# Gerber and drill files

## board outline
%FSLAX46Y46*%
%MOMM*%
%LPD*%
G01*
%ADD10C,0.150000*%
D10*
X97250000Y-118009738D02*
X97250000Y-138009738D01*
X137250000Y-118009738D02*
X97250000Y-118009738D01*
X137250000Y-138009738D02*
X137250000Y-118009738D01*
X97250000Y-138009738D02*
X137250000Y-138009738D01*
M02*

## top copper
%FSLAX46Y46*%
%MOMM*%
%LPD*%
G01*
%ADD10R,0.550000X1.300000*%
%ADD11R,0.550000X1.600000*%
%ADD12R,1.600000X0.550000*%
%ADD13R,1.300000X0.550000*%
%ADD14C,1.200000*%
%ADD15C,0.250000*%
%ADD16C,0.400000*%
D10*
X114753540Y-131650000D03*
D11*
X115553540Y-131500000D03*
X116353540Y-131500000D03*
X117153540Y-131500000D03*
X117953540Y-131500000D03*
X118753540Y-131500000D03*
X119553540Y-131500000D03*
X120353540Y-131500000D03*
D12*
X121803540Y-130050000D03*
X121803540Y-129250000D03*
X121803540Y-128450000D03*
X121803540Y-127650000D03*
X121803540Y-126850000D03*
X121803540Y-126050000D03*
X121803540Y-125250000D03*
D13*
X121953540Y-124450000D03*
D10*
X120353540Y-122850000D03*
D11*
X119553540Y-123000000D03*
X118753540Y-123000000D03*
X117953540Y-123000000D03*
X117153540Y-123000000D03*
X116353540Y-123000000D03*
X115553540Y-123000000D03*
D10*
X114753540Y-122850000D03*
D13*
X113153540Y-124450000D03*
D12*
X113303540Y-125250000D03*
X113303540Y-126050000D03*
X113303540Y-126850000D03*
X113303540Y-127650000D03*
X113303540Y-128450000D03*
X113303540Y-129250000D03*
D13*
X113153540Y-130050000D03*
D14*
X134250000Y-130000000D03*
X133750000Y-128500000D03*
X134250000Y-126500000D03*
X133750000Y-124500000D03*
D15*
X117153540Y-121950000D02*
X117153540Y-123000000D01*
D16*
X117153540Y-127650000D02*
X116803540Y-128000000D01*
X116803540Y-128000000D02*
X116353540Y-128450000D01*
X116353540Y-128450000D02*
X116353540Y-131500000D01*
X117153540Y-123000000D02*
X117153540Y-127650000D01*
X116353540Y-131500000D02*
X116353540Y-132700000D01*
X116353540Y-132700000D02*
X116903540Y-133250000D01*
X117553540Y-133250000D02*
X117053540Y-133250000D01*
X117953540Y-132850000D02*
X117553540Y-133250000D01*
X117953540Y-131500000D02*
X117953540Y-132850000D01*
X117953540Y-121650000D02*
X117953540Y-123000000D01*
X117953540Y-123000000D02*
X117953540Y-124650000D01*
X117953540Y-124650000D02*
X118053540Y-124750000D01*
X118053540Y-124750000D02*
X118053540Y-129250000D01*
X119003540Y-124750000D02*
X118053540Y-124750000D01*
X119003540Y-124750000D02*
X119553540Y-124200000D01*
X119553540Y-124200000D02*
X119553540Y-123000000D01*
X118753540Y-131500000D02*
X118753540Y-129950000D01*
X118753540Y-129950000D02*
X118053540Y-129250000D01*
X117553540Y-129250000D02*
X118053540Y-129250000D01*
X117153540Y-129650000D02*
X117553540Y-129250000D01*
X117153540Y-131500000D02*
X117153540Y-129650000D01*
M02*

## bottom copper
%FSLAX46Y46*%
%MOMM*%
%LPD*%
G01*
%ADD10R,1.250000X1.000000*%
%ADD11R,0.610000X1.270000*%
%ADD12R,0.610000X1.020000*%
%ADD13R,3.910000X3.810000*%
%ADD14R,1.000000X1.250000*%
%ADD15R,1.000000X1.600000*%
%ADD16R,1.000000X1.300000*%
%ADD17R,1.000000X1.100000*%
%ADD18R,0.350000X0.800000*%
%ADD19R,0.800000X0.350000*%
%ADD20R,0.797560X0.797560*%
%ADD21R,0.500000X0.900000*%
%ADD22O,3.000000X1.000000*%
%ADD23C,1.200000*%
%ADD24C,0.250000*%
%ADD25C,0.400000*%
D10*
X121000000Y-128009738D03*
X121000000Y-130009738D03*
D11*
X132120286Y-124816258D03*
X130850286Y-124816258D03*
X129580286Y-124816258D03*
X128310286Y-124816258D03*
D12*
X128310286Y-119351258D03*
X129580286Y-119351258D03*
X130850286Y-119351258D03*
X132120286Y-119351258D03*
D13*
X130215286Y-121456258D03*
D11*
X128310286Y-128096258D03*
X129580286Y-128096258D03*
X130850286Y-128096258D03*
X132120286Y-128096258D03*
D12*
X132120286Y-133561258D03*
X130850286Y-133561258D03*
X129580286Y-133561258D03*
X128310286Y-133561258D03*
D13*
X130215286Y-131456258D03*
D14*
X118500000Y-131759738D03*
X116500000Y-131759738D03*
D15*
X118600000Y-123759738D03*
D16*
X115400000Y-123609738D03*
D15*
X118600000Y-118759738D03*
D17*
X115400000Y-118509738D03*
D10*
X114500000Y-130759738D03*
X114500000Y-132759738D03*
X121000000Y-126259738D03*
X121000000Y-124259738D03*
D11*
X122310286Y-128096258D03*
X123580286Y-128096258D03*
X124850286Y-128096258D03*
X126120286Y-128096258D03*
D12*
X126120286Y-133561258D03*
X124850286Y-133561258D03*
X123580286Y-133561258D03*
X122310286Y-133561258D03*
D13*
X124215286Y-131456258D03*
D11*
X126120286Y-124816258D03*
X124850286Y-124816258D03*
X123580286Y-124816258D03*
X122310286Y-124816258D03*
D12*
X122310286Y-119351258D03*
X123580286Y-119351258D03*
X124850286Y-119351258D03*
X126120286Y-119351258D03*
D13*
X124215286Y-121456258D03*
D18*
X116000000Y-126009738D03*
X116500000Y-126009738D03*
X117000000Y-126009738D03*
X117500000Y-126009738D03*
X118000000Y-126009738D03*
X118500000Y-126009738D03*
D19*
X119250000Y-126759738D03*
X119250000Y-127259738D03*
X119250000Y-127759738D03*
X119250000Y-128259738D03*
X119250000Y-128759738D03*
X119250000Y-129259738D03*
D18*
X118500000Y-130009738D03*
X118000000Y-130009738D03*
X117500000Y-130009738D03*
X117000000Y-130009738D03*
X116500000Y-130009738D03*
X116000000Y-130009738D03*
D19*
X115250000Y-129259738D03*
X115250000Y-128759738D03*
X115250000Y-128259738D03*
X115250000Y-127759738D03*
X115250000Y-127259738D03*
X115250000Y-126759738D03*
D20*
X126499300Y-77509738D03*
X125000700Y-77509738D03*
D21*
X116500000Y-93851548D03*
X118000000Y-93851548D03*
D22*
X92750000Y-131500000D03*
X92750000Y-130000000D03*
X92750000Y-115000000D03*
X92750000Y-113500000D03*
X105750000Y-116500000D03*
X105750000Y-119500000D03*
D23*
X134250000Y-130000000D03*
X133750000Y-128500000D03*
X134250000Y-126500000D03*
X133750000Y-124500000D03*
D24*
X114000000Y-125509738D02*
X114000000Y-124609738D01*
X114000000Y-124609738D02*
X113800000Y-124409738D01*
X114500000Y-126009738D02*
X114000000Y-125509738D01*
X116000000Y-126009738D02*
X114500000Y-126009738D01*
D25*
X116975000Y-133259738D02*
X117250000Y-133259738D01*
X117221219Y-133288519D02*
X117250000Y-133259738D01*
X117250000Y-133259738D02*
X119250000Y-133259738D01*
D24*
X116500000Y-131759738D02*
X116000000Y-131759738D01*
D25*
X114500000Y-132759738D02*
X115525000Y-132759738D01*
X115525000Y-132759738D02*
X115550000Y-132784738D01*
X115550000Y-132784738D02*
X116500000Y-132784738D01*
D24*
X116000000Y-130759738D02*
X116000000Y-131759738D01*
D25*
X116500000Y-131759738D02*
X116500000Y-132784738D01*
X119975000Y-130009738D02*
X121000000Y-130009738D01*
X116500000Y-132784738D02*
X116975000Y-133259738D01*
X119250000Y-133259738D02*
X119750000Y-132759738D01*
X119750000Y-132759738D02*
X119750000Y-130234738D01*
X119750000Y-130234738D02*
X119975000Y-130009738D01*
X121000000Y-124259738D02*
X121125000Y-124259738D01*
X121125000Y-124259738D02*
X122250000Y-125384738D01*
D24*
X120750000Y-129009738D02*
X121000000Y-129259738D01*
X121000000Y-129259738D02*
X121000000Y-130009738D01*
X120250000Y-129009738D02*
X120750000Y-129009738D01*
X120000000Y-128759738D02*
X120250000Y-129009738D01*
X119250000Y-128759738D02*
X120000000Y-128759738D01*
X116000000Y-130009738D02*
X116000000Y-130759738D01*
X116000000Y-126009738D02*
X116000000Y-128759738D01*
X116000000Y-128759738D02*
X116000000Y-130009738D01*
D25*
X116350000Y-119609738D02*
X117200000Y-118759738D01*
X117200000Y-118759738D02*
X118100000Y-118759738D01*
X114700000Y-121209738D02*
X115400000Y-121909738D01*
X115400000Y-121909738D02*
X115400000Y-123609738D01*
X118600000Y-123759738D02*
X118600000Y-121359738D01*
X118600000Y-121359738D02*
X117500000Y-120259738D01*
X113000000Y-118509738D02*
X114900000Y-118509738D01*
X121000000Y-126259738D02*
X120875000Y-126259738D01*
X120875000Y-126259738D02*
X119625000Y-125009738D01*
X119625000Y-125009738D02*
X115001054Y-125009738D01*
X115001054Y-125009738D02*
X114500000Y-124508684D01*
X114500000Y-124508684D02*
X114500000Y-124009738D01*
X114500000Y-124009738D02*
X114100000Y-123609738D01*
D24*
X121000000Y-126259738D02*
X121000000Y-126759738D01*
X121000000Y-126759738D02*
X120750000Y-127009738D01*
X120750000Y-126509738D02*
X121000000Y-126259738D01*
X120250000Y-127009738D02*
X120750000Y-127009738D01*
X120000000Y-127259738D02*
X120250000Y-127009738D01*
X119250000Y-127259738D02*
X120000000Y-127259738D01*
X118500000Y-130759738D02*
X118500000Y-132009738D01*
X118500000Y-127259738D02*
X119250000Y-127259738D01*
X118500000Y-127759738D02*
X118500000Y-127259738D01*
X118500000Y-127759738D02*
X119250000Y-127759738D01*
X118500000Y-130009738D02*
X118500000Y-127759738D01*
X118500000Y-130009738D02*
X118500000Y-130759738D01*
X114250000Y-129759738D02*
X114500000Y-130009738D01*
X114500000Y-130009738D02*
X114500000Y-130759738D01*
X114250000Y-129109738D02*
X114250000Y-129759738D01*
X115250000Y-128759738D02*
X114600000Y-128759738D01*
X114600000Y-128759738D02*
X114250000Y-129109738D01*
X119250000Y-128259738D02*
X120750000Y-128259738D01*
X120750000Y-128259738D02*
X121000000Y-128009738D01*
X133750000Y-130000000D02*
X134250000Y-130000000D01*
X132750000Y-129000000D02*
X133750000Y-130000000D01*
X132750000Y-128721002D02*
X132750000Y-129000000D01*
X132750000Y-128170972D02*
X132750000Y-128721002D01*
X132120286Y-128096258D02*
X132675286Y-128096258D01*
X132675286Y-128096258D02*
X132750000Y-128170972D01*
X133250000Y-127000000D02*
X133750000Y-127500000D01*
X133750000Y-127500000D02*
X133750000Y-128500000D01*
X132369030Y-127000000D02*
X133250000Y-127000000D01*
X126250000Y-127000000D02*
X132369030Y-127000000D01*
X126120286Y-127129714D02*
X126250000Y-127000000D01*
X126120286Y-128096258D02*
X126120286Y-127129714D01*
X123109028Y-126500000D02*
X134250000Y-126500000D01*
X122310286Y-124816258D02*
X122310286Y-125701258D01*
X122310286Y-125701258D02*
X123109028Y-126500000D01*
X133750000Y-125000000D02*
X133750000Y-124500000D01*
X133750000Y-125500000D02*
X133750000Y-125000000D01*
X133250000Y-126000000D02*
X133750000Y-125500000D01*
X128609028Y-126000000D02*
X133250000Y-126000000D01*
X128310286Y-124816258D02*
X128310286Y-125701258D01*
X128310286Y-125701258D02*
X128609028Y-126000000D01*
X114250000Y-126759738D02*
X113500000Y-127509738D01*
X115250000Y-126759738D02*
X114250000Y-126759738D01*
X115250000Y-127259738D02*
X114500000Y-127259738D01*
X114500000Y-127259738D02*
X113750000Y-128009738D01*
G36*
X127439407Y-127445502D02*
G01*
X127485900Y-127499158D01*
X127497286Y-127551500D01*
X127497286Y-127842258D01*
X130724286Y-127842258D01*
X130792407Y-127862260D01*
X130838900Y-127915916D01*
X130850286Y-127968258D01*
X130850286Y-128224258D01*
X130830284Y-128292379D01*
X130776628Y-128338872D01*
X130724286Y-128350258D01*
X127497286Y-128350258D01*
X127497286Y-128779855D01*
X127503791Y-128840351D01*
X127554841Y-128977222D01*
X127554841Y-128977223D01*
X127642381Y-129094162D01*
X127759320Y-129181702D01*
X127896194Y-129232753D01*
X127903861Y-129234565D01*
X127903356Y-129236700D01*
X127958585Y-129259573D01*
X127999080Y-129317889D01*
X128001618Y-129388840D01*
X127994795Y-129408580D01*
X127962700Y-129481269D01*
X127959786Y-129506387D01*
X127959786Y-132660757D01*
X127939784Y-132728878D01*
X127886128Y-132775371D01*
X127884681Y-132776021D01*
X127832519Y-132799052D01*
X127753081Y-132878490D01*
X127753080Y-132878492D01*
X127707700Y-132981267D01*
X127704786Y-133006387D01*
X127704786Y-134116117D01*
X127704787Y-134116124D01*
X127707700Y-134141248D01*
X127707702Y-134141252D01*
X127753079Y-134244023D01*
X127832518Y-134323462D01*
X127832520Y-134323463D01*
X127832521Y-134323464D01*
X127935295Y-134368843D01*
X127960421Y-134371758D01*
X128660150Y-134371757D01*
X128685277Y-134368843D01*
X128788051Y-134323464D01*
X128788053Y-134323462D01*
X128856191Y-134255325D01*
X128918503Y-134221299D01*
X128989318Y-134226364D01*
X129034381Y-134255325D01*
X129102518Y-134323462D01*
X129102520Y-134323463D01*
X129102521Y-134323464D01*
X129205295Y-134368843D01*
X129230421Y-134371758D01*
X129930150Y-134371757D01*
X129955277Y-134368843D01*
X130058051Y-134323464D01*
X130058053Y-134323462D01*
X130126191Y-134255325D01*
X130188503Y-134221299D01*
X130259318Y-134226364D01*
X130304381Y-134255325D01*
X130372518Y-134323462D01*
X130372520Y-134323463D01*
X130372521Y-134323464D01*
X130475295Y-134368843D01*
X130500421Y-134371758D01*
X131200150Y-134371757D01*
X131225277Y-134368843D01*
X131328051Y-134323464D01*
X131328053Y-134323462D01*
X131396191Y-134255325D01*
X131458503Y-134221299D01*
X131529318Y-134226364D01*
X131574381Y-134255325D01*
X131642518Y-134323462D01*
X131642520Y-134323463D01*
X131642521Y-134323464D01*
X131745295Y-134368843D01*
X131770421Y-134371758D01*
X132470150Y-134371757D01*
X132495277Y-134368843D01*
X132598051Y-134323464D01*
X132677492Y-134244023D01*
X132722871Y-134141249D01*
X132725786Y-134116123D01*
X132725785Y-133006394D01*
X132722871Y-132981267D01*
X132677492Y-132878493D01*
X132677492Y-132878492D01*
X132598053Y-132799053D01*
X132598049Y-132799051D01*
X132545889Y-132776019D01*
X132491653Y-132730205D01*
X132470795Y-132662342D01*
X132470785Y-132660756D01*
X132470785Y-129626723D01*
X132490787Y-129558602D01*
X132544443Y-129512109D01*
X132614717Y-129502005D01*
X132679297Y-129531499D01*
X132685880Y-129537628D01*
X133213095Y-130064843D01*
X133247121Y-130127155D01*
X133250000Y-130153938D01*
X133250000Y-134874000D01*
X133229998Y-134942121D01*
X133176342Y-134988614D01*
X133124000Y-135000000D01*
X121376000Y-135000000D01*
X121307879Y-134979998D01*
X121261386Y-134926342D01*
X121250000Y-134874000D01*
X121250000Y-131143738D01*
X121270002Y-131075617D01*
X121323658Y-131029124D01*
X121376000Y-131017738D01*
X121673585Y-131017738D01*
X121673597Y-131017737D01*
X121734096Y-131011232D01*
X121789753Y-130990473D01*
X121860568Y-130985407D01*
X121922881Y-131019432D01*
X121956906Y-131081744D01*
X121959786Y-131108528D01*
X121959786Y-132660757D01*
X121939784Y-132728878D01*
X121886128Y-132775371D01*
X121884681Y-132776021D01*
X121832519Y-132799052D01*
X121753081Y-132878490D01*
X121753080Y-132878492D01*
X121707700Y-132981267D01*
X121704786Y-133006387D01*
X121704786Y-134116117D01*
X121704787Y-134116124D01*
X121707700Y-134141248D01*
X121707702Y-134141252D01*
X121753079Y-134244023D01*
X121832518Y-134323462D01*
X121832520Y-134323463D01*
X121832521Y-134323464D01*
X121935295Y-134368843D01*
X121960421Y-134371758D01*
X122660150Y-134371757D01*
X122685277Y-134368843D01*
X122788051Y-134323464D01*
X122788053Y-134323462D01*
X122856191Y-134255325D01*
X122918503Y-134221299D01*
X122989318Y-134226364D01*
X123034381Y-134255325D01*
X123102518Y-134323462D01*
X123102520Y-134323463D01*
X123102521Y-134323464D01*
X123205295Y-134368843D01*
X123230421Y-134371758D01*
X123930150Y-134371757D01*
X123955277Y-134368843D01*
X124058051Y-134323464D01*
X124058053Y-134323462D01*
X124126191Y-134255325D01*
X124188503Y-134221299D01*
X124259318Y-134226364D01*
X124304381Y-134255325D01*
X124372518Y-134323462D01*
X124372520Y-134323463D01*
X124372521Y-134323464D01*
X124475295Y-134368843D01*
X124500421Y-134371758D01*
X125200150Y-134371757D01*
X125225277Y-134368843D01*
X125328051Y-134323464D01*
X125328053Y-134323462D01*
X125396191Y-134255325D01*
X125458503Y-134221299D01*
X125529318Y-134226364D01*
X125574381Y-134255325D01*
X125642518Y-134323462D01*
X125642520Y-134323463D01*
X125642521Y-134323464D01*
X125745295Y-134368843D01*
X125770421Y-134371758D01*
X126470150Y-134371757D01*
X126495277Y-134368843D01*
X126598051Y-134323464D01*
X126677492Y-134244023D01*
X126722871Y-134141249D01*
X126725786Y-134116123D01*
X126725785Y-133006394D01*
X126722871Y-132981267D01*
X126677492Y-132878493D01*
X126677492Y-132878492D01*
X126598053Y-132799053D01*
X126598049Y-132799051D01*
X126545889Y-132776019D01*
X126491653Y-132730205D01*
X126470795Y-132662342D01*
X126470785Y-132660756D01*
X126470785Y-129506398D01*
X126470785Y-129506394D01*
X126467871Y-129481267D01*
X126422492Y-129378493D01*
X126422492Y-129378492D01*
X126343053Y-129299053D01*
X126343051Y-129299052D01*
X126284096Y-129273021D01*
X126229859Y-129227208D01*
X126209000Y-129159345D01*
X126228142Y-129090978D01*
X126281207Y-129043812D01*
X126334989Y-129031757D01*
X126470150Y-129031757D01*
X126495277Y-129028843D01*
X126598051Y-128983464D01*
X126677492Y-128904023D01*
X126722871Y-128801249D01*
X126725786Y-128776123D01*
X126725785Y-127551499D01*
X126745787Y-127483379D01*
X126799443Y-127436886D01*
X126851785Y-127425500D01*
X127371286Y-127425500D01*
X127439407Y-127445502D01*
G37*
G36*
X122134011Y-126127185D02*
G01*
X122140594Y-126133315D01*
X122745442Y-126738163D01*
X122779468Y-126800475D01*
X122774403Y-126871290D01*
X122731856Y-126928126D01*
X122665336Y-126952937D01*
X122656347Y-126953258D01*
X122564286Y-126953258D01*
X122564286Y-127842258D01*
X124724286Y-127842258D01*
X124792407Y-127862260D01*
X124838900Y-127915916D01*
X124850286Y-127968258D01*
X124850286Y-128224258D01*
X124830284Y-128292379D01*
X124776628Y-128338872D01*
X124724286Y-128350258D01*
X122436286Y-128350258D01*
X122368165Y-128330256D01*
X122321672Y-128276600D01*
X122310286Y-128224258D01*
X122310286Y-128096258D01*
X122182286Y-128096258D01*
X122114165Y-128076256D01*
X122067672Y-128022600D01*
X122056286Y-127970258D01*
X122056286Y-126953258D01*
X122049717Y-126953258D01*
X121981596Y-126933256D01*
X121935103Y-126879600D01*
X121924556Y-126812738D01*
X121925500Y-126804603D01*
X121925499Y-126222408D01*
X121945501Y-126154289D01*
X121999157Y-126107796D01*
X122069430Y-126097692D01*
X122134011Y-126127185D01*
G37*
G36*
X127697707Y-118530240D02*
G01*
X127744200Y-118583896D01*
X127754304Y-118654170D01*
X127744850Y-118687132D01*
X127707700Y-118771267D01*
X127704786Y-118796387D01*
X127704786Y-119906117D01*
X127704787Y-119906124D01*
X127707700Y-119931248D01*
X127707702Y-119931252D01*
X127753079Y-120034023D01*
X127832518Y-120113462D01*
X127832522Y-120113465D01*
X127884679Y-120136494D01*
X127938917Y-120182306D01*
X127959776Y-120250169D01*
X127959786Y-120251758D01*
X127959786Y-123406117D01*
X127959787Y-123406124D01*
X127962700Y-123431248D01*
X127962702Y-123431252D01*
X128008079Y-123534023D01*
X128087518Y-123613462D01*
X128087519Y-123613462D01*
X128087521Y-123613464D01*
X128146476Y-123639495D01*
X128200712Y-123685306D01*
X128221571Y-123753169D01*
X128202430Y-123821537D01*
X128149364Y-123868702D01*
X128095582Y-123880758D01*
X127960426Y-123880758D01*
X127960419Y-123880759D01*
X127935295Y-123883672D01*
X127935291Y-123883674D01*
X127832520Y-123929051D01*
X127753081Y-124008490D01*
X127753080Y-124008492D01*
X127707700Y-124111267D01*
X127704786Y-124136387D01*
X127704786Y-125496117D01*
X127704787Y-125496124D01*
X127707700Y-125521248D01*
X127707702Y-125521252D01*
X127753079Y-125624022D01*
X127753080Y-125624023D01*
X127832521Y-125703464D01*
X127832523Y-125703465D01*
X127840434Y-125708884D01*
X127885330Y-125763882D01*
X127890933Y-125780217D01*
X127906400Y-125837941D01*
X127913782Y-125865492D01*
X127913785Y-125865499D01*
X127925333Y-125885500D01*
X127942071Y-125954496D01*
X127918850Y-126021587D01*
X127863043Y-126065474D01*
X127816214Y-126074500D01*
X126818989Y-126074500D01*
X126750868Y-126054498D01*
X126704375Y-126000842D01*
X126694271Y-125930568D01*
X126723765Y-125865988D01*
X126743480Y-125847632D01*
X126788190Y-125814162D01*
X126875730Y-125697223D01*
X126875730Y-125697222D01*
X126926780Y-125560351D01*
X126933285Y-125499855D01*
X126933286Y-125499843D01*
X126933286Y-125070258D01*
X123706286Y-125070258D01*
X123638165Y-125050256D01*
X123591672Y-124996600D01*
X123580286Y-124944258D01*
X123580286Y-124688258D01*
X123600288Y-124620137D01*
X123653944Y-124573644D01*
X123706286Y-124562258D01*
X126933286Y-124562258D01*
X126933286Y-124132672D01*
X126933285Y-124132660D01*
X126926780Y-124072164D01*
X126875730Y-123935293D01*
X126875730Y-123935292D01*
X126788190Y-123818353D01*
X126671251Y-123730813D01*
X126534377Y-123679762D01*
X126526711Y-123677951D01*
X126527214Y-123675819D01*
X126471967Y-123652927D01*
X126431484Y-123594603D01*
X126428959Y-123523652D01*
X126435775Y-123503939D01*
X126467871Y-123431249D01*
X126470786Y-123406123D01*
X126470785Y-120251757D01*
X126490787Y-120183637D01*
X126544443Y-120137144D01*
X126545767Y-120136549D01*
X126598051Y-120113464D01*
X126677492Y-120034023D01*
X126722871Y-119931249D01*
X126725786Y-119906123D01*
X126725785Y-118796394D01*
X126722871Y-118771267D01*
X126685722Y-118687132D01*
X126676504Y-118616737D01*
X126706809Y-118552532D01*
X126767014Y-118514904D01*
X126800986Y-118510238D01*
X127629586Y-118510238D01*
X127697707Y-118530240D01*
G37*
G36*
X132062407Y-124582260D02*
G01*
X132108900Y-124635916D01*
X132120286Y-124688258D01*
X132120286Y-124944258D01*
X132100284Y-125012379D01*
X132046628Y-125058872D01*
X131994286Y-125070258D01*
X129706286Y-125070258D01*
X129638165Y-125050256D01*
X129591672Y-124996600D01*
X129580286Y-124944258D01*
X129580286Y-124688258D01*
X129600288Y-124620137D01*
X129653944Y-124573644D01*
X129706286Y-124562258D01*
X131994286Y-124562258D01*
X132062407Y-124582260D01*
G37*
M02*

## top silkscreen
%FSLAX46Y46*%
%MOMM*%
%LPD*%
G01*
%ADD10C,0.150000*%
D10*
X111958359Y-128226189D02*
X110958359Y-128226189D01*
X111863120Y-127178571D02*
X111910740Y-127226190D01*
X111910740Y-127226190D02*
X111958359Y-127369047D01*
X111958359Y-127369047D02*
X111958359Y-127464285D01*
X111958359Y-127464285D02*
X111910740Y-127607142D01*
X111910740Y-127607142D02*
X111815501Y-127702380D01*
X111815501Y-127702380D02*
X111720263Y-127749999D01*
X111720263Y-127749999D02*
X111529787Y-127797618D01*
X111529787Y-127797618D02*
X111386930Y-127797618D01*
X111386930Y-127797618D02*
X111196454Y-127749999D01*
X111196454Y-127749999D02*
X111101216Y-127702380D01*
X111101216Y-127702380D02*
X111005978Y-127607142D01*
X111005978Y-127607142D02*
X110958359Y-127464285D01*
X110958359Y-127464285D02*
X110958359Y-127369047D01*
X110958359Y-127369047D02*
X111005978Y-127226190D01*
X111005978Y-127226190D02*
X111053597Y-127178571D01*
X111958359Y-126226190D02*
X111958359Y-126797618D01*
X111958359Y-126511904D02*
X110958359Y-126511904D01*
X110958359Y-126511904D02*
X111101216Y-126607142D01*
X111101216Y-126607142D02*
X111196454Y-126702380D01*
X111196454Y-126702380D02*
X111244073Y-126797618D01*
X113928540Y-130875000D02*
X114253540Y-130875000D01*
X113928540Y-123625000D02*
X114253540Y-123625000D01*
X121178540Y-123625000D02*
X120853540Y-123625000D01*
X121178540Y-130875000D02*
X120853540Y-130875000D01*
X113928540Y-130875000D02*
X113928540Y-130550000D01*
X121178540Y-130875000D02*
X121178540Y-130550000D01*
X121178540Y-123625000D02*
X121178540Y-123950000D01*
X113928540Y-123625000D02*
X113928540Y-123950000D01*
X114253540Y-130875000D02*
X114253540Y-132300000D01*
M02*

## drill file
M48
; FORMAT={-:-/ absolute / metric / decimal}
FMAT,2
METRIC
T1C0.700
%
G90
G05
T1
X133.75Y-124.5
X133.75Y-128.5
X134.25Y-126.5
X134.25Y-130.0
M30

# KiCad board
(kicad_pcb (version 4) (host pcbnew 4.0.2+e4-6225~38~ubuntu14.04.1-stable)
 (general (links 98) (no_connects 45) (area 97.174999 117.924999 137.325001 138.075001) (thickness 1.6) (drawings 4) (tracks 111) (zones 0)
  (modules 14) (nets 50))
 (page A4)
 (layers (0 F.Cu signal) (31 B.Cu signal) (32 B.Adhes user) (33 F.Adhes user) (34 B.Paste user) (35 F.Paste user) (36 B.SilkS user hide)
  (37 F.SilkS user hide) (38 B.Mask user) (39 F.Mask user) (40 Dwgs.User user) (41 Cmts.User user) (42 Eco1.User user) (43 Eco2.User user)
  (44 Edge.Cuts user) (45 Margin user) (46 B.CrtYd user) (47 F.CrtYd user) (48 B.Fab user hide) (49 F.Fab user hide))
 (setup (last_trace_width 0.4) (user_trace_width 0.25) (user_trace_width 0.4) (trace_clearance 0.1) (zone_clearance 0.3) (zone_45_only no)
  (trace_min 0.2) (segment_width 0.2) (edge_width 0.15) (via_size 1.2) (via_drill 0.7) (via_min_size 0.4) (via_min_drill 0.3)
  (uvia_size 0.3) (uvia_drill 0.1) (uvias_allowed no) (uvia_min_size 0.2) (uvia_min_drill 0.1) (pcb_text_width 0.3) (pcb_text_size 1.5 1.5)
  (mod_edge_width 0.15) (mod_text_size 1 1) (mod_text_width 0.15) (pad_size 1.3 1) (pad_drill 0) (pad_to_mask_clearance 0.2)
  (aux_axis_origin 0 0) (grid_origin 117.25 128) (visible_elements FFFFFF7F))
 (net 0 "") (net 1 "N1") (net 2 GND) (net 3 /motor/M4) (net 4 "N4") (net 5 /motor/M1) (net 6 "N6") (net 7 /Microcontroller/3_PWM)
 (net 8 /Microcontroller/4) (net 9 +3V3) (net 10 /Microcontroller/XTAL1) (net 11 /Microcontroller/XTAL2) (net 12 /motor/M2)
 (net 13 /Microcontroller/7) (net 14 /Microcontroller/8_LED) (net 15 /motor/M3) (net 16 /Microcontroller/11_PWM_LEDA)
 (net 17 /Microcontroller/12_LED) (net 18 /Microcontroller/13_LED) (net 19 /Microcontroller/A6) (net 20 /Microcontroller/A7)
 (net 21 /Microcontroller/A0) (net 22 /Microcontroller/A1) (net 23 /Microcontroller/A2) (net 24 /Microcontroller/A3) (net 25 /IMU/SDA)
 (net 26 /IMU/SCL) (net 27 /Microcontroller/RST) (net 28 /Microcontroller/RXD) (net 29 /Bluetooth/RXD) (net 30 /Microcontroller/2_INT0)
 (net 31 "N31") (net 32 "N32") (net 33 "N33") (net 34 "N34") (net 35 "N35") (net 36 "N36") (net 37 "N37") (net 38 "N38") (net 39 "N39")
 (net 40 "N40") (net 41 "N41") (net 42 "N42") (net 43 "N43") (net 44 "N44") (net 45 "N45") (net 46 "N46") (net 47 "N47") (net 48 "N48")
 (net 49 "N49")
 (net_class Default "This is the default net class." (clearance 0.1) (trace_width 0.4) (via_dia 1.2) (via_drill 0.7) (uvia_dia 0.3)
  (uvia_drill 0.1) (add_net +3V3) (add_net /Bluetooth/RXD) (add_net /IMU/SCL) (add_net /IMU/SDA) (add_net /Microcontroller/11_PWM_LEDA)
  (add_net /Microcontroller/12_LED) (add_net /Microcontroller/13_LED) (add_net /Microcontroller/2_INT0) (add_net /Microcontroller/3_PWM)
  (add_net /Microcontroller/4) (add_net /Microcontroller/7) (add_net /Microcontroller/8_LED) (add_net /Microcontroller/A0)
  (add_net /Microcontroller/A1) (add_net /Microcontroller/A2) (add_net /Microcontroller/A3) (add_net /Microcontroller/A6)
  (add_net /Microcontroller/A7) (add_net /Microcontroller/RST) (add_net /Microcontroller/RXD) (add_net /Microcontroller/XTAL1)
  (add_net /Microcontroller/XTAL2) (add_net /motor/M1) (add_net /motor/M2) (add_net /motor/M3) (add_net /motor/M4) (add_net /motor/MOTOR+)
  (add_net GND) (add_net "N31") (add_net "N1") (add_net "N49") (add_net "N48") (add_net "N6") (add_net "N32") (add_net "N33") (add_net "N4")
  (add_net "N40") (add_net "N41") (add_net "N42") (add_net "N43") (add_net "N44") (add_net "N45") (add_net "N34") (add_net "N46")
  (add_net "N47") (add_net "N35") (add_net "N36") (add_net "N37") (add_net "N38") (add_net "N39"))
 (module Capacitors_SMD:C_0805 (layer B.Cu) (at 121 129.009738 270)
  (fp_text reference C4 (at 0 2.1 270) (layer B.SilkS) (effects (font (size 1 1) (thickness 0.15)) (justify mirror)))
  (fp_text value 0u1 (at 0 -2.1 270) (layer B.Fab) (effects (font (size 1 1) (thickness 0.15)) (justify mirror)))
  (pad 1 smd rect (at -1 0 270) (size 1 1.25) (layers B.Cu B.Paste B.Mask) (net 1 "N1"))
  (pad 2 smd rect (at 1 0 270) (size 1 1.25) (layers B.Cu B.Paste B.Mask) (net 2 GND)))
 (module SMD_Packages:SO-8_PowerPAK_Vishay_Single (layer B.Cu) (at 130.215286 122.146258 90)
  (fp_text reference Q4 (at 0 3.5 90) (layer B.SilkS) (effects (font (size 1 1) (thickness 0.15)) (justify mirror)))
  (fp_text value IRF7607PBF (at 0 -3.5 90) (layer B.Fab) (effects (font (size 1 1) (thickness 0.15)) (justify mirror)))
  (pad 1 smd rect (at -2.67 1.905 90) (size 1.27 0.61) (layers B.Cu B.Paste B.Mask) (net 2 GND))
  (pad 2 smd rect (at -2.67 0.635 90) (size 1.27 0.61) (layers B.Cu B.Paste B.Mask) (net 2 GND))
  (pad 3 smd rect (at -2.67 -0.635 90) (size 1.27 0.61) (layers B.Cu B.Paste B.Mask) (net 2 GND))
  (pad 4 smd rect (at -2.67 -1.905 90) (size 1.27 0.61) (layers B.Cu B.Paste B.Mask) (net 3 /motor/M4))
  (pad 5 smd rect (at 2.795 -1.905 90) (size 1.02 0.61) (layers B.Cu B.Paste B.Mask) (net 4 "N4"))
  (pad 5 smd rect (at 2.795 -0.635 90) (size 1.02 0.61) (layers B.Cu B.Paste B.Mask) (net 4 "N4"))
  (pad 5 smd rect (at 2.795 0.635 90) (size 1.02 0.61) (layers B.Cu B.Paste B.Mask) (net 4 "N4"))
  (pad 5 smd rect (at 2.795 1.905 90) (size 1.02 0.61) (layers B.Cu B.Paste B.Mask) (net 4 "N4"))
  (pad 5 smd rect (at 0.69 0 90) (size 3.81 3.91) (layers B.Cu B.Paste B.Mask) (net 4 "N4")))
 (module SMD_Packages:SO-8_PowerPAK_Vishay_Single (layer B.Cu) (at 130.215286 130.766258 270)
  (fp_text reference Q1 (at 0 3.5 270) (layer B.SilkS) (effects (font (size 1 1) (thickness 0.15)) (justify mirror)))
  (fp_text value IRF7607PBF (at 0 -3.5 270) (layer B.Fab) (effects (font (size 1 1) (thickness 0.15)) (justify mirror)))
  (pad 1 smd rect (at -2.67 1.905 270) (size 1.27 0.61) (layers B.Cu B.Paste B.Mask) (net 2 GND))
  (pad 2 smd rect (at -2.67 0.635 270) (size 1.27 0.61) (layers B.Cu B.Paste B.Mask) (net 2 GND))
  (pad 3 smd rect (at -2.67 -0.635 270) (size 1.27 0.61) (layers B.Cu B.Paste B.Mask) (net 2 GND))
  (pad 4 smd rect (at -2.67 -1.905 270) (size 1.27 0.61) (layers B.Cu B.Paste B.Mask) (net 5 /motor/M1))
  (pad 5 smd rect (at 2.795 -1.905 270) (size 1.02 0.61) (layers B.Cu B.Paste B.Mask) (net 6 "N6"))
  (pad 5 smd rect (at 2.795 -0.635 270) (size 1.02 0.61) (layers B.Cu B.Paste B.Mask) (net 6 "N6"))
  (pad 5 smd rect (at 2.795 0.635 270) (size 1.02 0.61) (layers B.Cu B.Paste B.Mask) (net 6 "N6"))
  (pad 5 smd rect (at 2.795 1.905 270) (size 1.02 0.61) (layers B.Cu B.Paste B.Mask) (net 6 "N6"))
  (pad 5 smd rect (at 0.69 0 270) (size 3.81 3.91) (layers B.Cu B.Paste B.Mask) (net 6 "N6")))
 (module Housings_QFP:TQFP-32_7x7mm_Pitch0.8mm (layer F.Cu) (at 117.55354 127.25 90)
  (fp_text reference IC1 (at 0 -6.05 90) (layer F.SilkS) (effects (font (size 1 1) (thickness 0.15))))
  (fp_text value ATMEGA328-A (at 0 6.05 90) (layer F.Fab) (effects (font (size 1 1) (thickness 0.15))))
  (fp_line (start -3.625 -3.625) (end -3.625 -3.3) (layer F.SilkS) (width 0.15))
  (fp_line (start 3.625 -3.625) (end 3.625 -3.3) (layer F.SilkS) (width 0.15))
  (fp_line (start 3.625 3.625) (end 3.625 3.3) (layer F.SilkS) (width 0.15))
  (fp_line (start -3.625 3.625) (end -3.625 3.3) (layer F.SilkS) (width 0.15))
  (fp_line (start -3.625 -3.625) (end -3.3 -3.625) (layer F.SilkS) (width 0.15))
  (fp_line (start -3.625 3.625) (end -3.3 3.625) (layer F.SilkS) (width 0.15))
  (fp_line (start 3.625 3.625) (end 3.3 3.625) (layer F.SilkS) (width 0.15))
  (fp_line (start 3.625 -3.625) (end 3.3 -3.625) (layer F.SilkS) (width 0.15))
  (fp_line (start -3.625 -3.3) (end -5.05 -3.3) (layer F.SilkS) (width 0.15))
  (pad 1 smd rect (at -4.4 -2.8 90) (size 1.3 0.55) (layers F.Cu F.Paste F.Mask) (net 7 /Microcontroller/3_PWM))
  (pad 2 smd rect (at -4.25 -2 90) (size 1.6 0.55) (layers F.Cu F.Paste F.Mask) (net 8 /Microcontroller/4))
  (pad 3 smd rect (at -4.25 -1.2 90) (size 1.6 0.55) (layers F.Cu F.Paste F.Mask) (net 2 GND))
  (pad 4 smd rect (at -4.25 -0.4 90) (size 1.6 0.55) (layers F.Cu F.Paste F.Mask) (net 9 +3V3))
  (pad 5 smd rect (at -4.25 0.4 90) (size 1.6 0.55) (layers F.Cu F.Paste F.Mask) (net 2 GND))
  (pad 6 smd rect (at -4.25 1.2 90) (size 1.6 0.55) (layers F.Cu F.Paste F.Mask) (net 9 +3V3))
  (pad 7 smd rect (at -4.25 2 90) (size 1.6 0.55) (layers F.Cu F.Paste F.Mask) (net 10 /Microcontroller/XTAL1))
  (pad 8 smd rect (at -4.25 2.8 90) (size 1.6 0.55) (layers F.Cu F.Paste F.Mask) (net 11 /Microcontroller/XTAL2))
  (pad 9 smd rect (at -2.8 4.25 180) (size 1.6 0.55) (layers F.Cu F.Paste F.Mask) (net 5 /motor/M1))
  (pad 10 smd rect (at -2 4.25 180) (size 1.6 0.55) (layers F.Cu F.Paste F.Mask) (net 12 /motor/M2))
  (pad 11 smd rect (at -1.2 4.25 180) (size 1.6 0.55) (layers F.Cu F.Paste F.Mask) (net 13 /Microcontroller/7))
  (pad 12 smd rect (at -0.4 4.25 180) (size 1.6 0.55) (layers F.Cu F.Paste F.Mask) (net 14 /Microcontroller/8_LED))
  (pad 13 smd rect (at 0.4 4.25 180) (size 1.6 0.55) (layers F.Cu F.Paste F.Mask) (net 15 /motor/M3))
  (pad 14 smd rect (at 1.2 4.25 180) (size 1.6 0.55) (layers F.Cu F.Paste F.Mask) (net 3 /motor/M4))
  (pad 15 smd rect (at 2 4.25 180) (size 1.6 0.55) (layers F.Cu F.Paste F.Mask) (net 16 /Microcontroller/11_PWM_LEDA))
  (pad 16 smd rect (at 2.8 4.4 180) (size 1.3 0.55) (layers F.Cu F.Paste F.Mask) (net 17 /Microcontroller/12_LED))
  (pad 17 smd rect (at 4.4 2.8 90) (size 1.3 0.55) (layers F.Cu F.Paste F.Mask) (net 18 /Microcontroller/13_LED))
  (pad 18 smd rect (at 4.25 2 90) (size 1.6 0.55) (layers F.Cu F.Paste F.Mask) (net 9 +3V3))
  (pad 19 smd rect (at 4.25 1.2 90) (size 1.6 0.55) (layers F.Cu F.Paste F.Mask) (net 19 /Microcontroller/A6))
  (pad 20 smd rect (at 4.25 0.4 90) (size 1.6 0.55) (layers F.Cu F.Paste F.Mask) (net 9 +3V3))
  (pad 21 smd rect (at 4.25 -0.4 90) (size 1.6 0.55) (layers F.Cu F.Paste F.Mask) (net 2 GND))
  (pad 22 smd rect (at 4.25 -1.2 90) (size 1.6 0.55) (layers F.Cu F.Paste F.Mask) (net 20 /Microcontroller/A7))
  (pad 23 smd rect (at 4.25 -2 90) (size 1.6 0.55) (layers F.Cu F.Paste F.Mask) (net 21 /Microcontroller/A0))
  (pad 24 smd rect (at 4.4 -2.8 90) (size 1.3 0.55) (layers F.Cu F.Paste F.Mask) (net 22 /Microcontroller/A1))
  (pad 25 smd rect (at 2.8 -4.4 180) (size 1.3 0.55) (layers F.Cu F.Paste F.Mask) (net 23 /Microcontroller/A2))
  (pad 26 smd rect (at 2 -4.25 180) (size 1.6 0.55) (layers F.Cu F.Paste F.Mask) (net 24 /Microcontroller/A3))
  (pad 27 smd rect (at 1.2 -4.25 180) (size 1.6 0.55) (layers F.Cu F.Paste F.Mask) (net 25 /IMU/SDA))
  (pad 28 smd rect (at 0.4 -4.25 180) (size 1.6 0.55) (layers F.Cu F.Paste F.Mask) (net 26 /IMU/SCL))
  (pad 29 smd rect (at -0.4 -4.25 180) (size 1.6 0.55) (layers F.Cu F.Paste F.Mask) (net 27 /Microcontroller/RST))
  (pad 30 smd rect (at -1.2 -4.25 180) (size 1.6 0.55) (layers F.Cu F.Paste F.Mask) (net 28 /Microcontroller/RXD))
  (pad 31 smd rect (at -2 -4.25 180) (size 1.6 0.55) (layers F.Cu F.Paste F.Mask) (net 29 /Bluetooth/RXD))
  (pad 32 smd rect (at -2.8 -4.4 180) (size 1.3 0.55) (layers F.Cu F.Paste F.Mask) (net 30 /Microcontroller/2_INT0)))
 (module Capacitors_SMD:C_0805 (layer B.Cu) (at 117.5 131.759738 180)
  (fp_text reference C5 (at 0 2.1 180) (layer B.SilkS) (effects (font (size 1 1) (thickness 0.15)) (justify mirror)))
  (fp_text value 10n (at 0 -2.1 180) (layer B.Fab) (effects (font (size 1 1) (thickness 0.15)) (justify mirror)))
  (pad 1 smd rect (at -1 0 180) (size 1 1.25) (layers B.Cu B.Paste B.Mask) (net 9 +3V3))
  (pad 2 smd rect (at 1 0 180) (size 1 1.25) (layers B.Cu B.Paste B.Mask) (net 2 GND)))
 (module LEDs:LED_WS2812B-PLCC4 (layer B.Cu) (at 117 121.259738 270)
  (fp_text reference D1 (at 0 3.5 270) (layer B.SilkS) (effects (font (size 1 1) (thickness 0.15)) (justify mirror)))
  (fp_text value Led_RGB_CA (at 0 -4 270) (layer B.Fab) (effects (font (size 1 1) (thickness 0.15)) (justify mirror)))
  (pad 3 smd rect (at 2.5 -1.6 270) (size 1.6 1) (layers B.Cu B.Paste B.Mask) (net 14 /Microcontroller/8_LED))
  (pad 4 smd rect (at 2.35 1.6 270) (size 1.3 1) (layers B.Cu B.Paste B.Mask) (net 18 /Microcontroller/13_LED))
  (pad 2 smd rect (at -2.5 -1.6 270) (size 1.6 1) (layers B.Cu B.Paste B.Mask) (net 17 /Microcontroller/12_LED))
  (pad 1 smd rect (at -2.75 1.6 270) (size 1.1 1) (layers B.Cu B.Paste B.Mask) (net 16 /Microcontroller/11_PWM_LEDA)))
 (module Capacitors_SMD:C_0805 (layer B.Cu) (at 114.5 131.759738 270)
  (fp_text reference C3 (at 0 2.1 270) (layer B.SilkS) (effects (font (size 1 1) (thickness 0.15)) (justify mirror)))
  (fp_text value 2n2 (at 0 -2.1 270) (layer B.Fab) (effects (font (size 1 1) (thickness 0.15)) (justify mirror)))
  (pad 1 smd rect (at -1 0 270) (size 1 1.25) (layers B.Cu B.Paste B.Mask) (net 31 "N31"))
  (pad 2 smd rect (at 1 0 270) (size 1 1.25) (layers B.Cu B.Paste B.Mask) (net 2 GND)))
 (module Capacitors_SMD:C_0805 (layer B.Cu) (at 121 125.259738 90)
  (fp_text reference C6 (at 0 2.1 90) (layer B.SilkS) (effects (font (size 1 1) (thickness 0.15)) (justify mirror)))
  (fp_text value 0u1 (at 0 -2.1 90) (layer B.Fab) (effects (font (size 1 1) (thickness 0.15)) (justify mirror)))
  (pad 1 smd rect (at -1 0 90) (size 1 1.25) (layers B.Cu B.Paste B.Mask) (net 9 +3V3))
  (pad 2 smd rect (at 1 0 90) (size 1 1.25) (layers B.Cu B.Paste B.Mask) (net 2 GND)))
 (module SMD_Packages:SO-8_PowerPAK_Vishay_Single (layer B.Cu) (at 124.215286 130.766258 270)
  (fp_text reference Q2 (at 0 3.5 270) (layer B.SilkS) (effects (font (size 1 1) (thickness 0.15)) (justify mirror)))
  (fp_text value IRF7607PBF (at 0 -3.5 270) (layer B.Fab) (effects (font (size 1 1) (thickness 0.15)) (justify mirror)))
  (pad 1 smd rect (at -2.67 1.905 270) (size 1.27 0.61) (layers B.Cu B.Paste B.Mask) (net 2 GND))
  (pad 2 smd rect (at -2.67 0.635 270) (size 1.27 0.61) (layers B.Cu B.Paste B.Mask) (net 2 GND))
  (pad 3 smd rect (at -2.67 -0.635 270) (size 1.27 0.61) (layers B.Cu B.Paste B.Mask) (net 2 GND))
  (pad 4 smd rect (at -2.67 -1.905 270) (size 1.27 0.61) (layers B.Cu B.Paste B.Mask) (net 12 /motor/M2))
  (pad 5 smd rect (at 2.795 -1.905 270) (size 1.02 0.61) (layers B.Cu B.Paste B.Mask) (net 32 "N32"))
  (pad 5 smd rect (at 2.795 -0.635 270) (size 1.02 0.61) (layers B.Cu B.Paste B.Mask) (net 32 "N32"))
  (pad 5 smd rect (at 2.795 0.635 270) (size 1.02 0.61) (layers B.Cu B.Paste B.Mask) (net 32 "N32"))
  (pad 5 smd rect (at 2.795 1.905 270) (size 1.02 0.61) (layers B.Cu B.Paste B.Mask) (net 32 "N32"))
  (pad 5 smd rect (at 0.69 0 270) (size 3.81 3.91) (layers B.Cu B.Paste B.Mask) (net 32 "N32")))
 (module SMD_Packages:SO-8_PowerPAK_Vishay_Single (layer B.Cu) (at 124.215286 122.146258 90)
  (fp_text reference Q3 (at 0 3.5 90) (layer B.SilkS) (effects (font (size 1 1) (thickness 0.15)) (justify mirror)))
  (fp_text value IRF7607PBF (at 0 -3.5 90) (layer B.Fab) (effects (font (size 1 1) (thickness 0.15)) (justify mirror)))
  (pad 1 smd rect (at -2.67 1.905 90) (size 1.27 0.61) (layers B.Cu B.Paste B.Mask) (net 2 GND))
  (pad 2 smd rect (at -2.67 0.635 90) (size 1.27 0.61) (layers B.Cu B.Paste B.Mask) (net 2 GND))
  (pad 3 smd rect (at -2.67 -0.635 90) (size 1.27 0.61) (layers B.Cu B.Paste B.Mask) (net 2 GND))
  (pad 4 smd rect (at -2.67 -1.905 90) (size 1.27 0.61) (layers B.Cu B.Paste B.Mask) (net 15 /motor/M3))
  (pad 5 smd rect (at 2.795 -1.905 90) (size 1.02 0.61) (layers B.Cu B.Paste B.Mask) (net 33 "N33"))
  (pad 5 smd rect (at 2.795 -0.635 90) (size 1.02 0.61) (layers B.Cu B.Paste B.Mask) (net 33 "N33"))
  (pad 5 smd rect (at 2.795 0.635 90) (size 1.02 0.61) (layers B.Cu B.Paste B.Mask) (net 33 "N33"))
  (pad 5 smd rect (at 2.795 1.905 90) (size 1.02 0.61) (layers B.Cu B.Paste B.Mask) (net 33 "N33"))
  (pad 5 smd rect (at 0.69 0 90) (size 3.81 3.91) (layers B.Cu B.Paste B.Mask) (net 33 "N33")))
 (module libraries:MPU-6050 (layer B.Cu) (at 117.25 128.009738 270)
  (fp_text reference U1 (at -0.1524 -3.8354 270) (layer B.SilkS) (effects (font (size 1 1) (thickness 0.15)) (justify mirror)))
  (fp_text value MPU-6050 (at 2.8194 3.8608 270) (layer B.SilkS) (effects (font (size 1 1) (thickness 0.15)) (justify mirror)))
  (pad 1 smd rect (at -2 1.25 270) (size 0.8 0.35) (layers B.Cu B.Paste B.Mask) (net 2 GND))
  (pad 2 smd rect (at -2 0.75 270) (size 0.8 0.35) (layers B.Cu B.Paste B.Mask) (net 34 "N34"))
  (pad 3 smd rect (at -2 0.25 270) (size 0.8 0.35) (layers B.Cu B.Paste B.Mask) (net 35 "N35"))
  (pad 4 smd rect (at -2 -0.25 270) (size 0.8 0.35) (layers B.Cu B.Paste B.Mask) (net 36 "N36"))
  (pad 5 smd rect (at -2 -0.75 270) (size 0.8 0.35) (layers B.Cu B.Paste B.Mask) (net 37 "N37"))
  (pad 6 smd rect (at -2 -1.25 270) (size 0.8 0.35) (layers B.Cu B.Paste B.Mask) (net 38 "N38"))
  (pad 7 smd rect (at -1.25 -2 270) (size 0.35 0.8) (layers B.Cu B.Paste B.Mask) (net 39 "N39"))
  (pad 8 smd rect (at -0.75 -2 270) (size 0.35 0.8) (layers B.Cu B.Paste B.Mask) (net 9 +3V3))
  (pad 9 smd rect (at -0.25 -2 270) (size 0.35 0.8) (layers B.Cu B.Paste B.Mask) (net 9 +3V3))
  (pad 10 smd rect (at 0.25 -2 270) (size 0.35 0.8) (layers B.Cu B.Paste B.Mask) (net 1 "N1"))
  (pad 11 smd rect (at 0.75 -2 270) (size 0.35 0.8) (layers B.Cu B.Paste B.Mask) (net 2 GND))
  (pad 12 smd rect (at 1.25 -2 270) (size 0.35 0.8) (layers B.Cu B.Paste B.Mask) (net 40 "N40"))
  (pad 13 smd rect (at 2 -1.25 270) (size 0.8 0.35) (layers B.Cu B.Paste B.Mask) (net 9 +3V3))
  (pad 14 smd rect (at 2 -0.75 270) (size 0.8 0.35) (layers B.Cu B.Paste B.Mask) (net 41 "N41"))
  (pad 15 smd rect (at 2 -0.25 270) (size 0.8 0.35) (layers B.Cu B.Paste B.Mask) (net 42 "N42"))
  (pad 16 smd rect (at 2 0.25 270) (size 0.8 0.35) (layers B.Cu B.Paste B.Mask) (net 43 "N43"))
  (pad 17 smd rect (at 2 0.75 270) (size 0.8 0.35) (layers B.Cu B.Paste B.Mask) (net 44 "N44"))
  (pad 18 smd rect (at 2 1.25 270) (size 0.8 0.35) (layers B.Cu B.Paste B.Mask) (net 2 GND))
  (pad 19 smd rect (at 1.25 2 270) (size 0.35 0.8) (layers B.Cu B.Paste B.Mask) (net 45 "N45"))
  (pad 20 smd rect (at 0.75 2 270) (size 0.35 0.8) (layers B.Cu B.Paste B.Mask) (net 31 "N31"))
  (pad 21 smd rect (at 0.25 2 270) (size 0.35 0.8) (layers B.Cu B.Paste B.Mask) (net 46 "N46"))
  (pad 22 smd rect (at -0.25 2 270) (size 0.35 0.8) (layers B.Cu B.Paste B.Mask) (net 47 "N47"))
  (pad 23 smd rect (at -0.75 2 270) (size 0.35 0.8) (layers B.Cu B.Paste B.Mask) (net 26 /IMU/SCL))
  (pad 24 smd rect (at -1.25 2 270) (size 0.35 0.8) (layers B.Cu B.Paste B.Mask) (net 25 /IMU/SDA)))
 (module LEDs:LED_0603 (layer B.Cu) (at 125.75 77.509738)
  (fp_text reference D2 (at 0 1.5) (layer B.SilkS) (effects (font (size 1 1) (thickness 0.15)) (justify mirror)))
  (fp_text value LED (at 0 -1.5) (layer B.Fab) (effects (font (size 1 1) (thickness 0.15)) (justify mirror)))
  (pad 2 smd rect (at 0.7493 0 180) (size 0.79756 0.79756) (layers B.Cu B.Paste B.Mask) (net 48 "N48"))
  (pad 1 smd rect (at -0.7493 0 180) (size 0.79756 0.79756) (layers B.Cu B.Paste B.Mask) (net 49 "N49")))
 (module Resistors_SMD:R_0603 (layer B.Cu) (at 117.25 93.851548)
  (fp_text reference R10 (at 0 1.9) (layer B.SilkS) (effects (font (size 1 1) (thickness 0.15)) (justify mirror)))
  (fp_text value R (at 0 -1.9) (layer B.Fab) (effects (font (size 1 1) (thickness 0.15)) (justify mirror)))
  (pad 1 smd rect (at -0.75 0) (size 0.5 0.9) (layers B.Cu B.Paste B.Mask) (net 49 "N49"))
  (pad 2 smd rect (at 0.75 0) (size 0.5 0.9) (layers B.Cu B.Paste B.Mask) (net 2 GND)))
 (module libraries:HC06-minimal (layer B.Cu) (at 98.75 122.5)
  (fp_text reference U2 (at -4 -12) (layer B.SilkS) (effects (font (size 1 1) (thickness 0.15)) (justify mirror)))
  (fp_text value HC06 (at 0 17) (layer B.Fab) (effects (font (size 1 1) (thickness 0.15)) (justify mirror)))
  (pad 1 smd oval (at -6 9) (size 3 1) (layers B.Cu B.Paste B.Mask) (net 28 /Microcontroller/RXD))
  (pad 2 smd oval (at -6 7.5) (size 3 1) (layers B.Cu B.Paste B.Mask) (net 29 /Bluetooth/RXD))
  (pad 12 smd oval (at -6 -7.5) (size 3 1) (layers B.Cu B.Paste B.Mask) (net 9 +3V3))
  (pad 13 smd oval (at -6 -9) (size 3 1) (layers B.Cu B.Paste B.Mask) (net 2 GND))
  (pad 24 smd oval (at 7 -6) (size 3 1) (layers B.Cu B.Paste B.Mask) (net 48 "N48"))
  (pad 26 smd oval (at 7 -3) (size 3 1) (layers B.Cu B.Paste B.Mask) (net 2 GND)))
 (gr_line (start 97.25 118.009738) (end 97.25 138.009738) (layer Edge.Cuts) (width 0.15))
 (gr_line (start 137.25 118.009738) (end 97.25 118.009738) (layer Edge.Cuts) (width 0.15))
 (gr_line (start 137.25 138.009738) (end 137.25 118.009738) (layer Edge.Cuts) (width 0.15))
 (gr_line (start 97.25 138.009738) (end 137.25 138.009738) (layer Edge.Cuts) (width 0.15))
 (segment (start 114 125.509738) (end 114 124.609738) (width 0.25) (layer B.Cu) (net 2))
 (segment (start 114 124.609738) (end 113.8 124.409738) (width 0.25) (layer B.Cu) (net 2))
 (segment (start 114.5 126.009738) (end 114 125.509738) (width 0.25) (layer B.Cu) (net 2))
 (segment (start 116 126.009738) (end 114.5 126.009738) (width 0.25) (layer B.Cu) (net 2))
 (segment (start 117.15354 121.95) (end 117.15354 123) (width 0.25) (layer F.Cu) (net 2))
 (segment (start 116.975 133.259738) (end 117.25 133.259738) (width 0.4) (layer B.Cu) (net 2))
 (segment (start 117.221219 133.288519) (end 117.25 133.259738) (width 0.4) (layer B.Cu) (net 2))
 (segment (start 117.25 133.259738) (end 119.25 133.259738) (width 0.4) (layer B.Cu) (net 2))
 (segment (start 117.15354 127.65) (end 116.80354 128) (width 0.4) (layer F.Cu) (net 2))
 (segment (start 116.80354 128) (end 116.35354 128.45) (width 0.4) (layer F.Cu) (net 2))
 (segment (start 116.35354 128.45) (end 116.35354 131.5) (width 0.4) (layer F.Cu) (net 2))
 (segment (start 117.15354 123) (end 117.15354 127.65) (width 0.4) (layer F.Cu) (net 2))
 (segment (start 116.35354 131.5) (end 116.35354 132.7) (width 0.4) (layer F.Cu) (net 2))
 (segment (start 116.35354 132.7) (end 116.90354 133.25) (width 0.4) (layer F.Cu) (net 2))
 (segment (start 117.55354 133.25) (end 117.05354 133.25) (width 0.4) (layer F.Cu) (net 2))
 (segment (start 117.95354 132.85) (end 117.55354 133.25) (width 0.4) (layer F.Cu) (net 2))
 (segment (start 117.95354 131.5) (end 117.95354 132.85) (width 0.4) (layer F.Cu) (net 2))
 (segment (start 116.5 131.759738) (end 116 131.759738) (width 0.25) (layer B.Cu) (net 2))
 (segment (start 114.5 132.759738) (end 115.525 132.759738) (width 0.4) (layer B.Cu) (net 2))
 (segment (start 115.525 132.759738) (end 115.55 132.784738) (width 0.4) (layer B.Cu) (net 2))
 (segment (start 115.55 132.784738) (end 116.5 132.784738) (width 0.4) (layer B.Cu) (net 2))
 (segment (start 116 130.759738) (end 116 131.759738) (width 0.25) (layer B.Cu) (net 2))
 (segment (start 116.5 131.759738) (end 116.5 132.784738) (width 0.4) (layer B.Cu) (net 2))
 (segment (start 119.975 130.009738) (end 121 130.009738) (width 0.4) (layer B.Cu) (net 2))
 (segment (start 116.5 132.784738) (end 116.975 133.259738) (width 0.4) (layer B.Cu) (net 2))
 (segment (start 119.25 133.259738) (end 119.75 132.759738) (width 0.4) (layer B.Cu) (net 2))
 (segment (start 119.75 132.759738) (end 119.75 130.234738) (width 0.4) (layer B.Cu) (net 2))
 (segment (start 119.75 130.234738) (end 119.975 130.009738) (width 0.4) (layer B.Cu) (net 2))
 (segment (start 121 124.259738) (end 121.125 124.259738) (width 0.4) (layer B.Cu) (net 2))
 (segment (start 121.125 124.259738) (end 122.25 125.384738) (width 0.4) (layer B.Cu) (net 2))
 (segment (start 120.75 129.009738) (end 121 129.259738) (width 0.25) (layer B.Cu) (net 2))
 (segment (start 121 129.259738) (end 121 130.009738) (width 0.25) (layer B.Cu) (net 2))
 (segment (start 120.25 129.009738) (end 120.75 129.009738) (width 0.25) (layer B.Cu) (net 2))
 (segment (start 120 128.759738) (end 120.25 129.009738) (width 0.25) (layer B.Cu) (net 2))
 (segment (start 119.25 128.759738) (end 120 128.759738) (width 0.25) (layer B.Cu) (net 2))
 (segment (start 116 130.009738) (end 116 130.759738) (width 0.25) (layer B.Cu) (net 2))
 (segment (start 116 126.009738) (end 116 128.759738) (width 0.25) (layer B.Cu) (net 2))
 (segment (start 116 128.759738) (end 116 130.009738) (width 0.25) (layer B.Cu) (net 2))
 (segment (start 116.35 119.609738) (end 117.2 118.759738) (width 0.4) (layer B.Cu) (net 17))
 (segment (start 117.2 118.759738) (end 118.1 118.759738) (width 0.4) (layer B.Cu) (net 17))
 (segment (start 114.7 121.209738) (end 115.4 121.909738) (width 0.4) (layer B.Cu) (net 18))
 (segment (start 115.4 121.909738) (end 115.4 123.609738) (width 0.4) (layer B.Cu) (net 18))
 (segment (start 118.6 123.759738) (end 118.6 121.359738) (width 0.4) (layer B.Cu) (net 14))
 (segment (start 118.6 121.359738) (end 117.5 120.259738) (width 0.4) (layer B.Cu) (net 14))
 (segment (start 113 118.509738) (end 114.9 118.509738) (width 0.4) (layer B.Cu) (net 16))
 (segment (start 121 126.259738) (end 120.875 126.259738) (width 0.4) (layer B.Cu) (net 9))
 (segment (start 120.875 126.259738) (end 119.625 125.009738) (width 0.4) (layer B.Cu) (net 9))
 (segment (start 119.625 125.009738) (end 115.001054 125.009738) (width 0.4) (layer B.Cu) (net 9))
 (segment (start 117.95354 121.65) (end 117.95354 123) (width 0.4) (layer F.Cu) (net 9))
 (segment (start 115.001054 125.009738) (end 114.5 124.508684) (width 0.4) (layer B.Cu) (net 9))
 (segment (start 114.5 124.508684) (end 114.5 124.009738) (width 0.4) (layer B.Cu) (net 9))
 (segment (start 114.5 124.009738) (end 114.1 123.609738) (width 0.4) (layer B.Cu) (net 9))
 (segment (start 117.95354 123) (end 117.95354 124.65) (width 0.4) (layer F.Cu) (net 9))
 (segment (start 117.95354 124.65) (end 118.05354 124.75) (width 0.4) (layer F.Cu) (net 9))
 (segment (start 118.05354 124.75) (end 118.05354 129.25) (width 0.4) (layer F.Cu) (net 9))
 (segment (start 119.00354 124.75) (end 118.05354 124.75) (width 0.4) (layer F.Cu) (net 9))
 (segment (start 119.00354 124.75) (end 119.55354 124.2) (width 0.4) (layer F.Cu) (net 9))
 (segment (start 119.55354 124.2) (end 119.55354 123) (width 0.4) (layer F.Cu) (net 9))
 (segment (start 118.75354 131.5) (end 118.75354 129.95) (width 0.4) (layer F.Cu) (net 9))
 (segment (start 118.75354 129.95) (end 118.05354 129.25) (width 0.4) (layer F.Cu) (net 9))
 (segment (start 117.55354 129.25) (end 118.05354 129.25) (width 0.4) (layer F.Cu) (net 9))
 (segment (start 117.15354 129.65) (end 117.55354 129.25) (width 0.4) (layer F.Cu) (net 9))
 (segment (start 117.15354 131.5) (end 117.15354 129.65) (width 0.4) (layer F.Cu) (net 9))
 (segment (start 121 126.259738) (end 121 126.759738) (width 0.25) (layer B.Cu) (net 9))
 (segment (start 121 126.759738) (end 120.75 127.009738) (width 0.25) (layer B.Cu) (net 9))
 (segment (start 120.75 126.509738) (end 121 126.259738) (width 0.25) (layer B.Cu) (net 9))
 (segment (start 120.25 127.009738) (end 120.75 127.009738) (width 0.25) (layer B.Cu) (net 9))
 (segment (start 120 127.259738) (end 120.25 127.009738) (width 0.25) (layer B.Cu) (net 9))
 (segment (start 119.25 127.259738) (end 120 127.259738) (width 0.25) (layer B.Cu) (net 9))
 (segment (start 118.5 130.759738) (end 118.5 132.009738) (width 0.25) (layer B.Cu) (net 9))
 (segment (start 118.5 127.259738) (end 119.25 127.259738) (width 0.25) (layer B.Cu) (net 9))
 (segment (start 118.5 127.759738) (end 118.5 127.259738) (width 0.25) (layer B.Cu) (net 9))
 (segment (start 118.5 127.759738) (end 119.25 127.759738) (width 0.25) (layer B.Cu) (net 9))
 (segment (start 118.5 130.009738) (end 118.5 127.759738) (width 0.25) (layer B.Cu) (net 9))
 (segment (start 118.5 130.009738) (end 118.5 130.759738) (width 0.25) (layer B.Cu) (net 9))
 (segment (start 114.25 129.759738) (end 114.5 130.009738) (width 0.25) (layer B.Cu) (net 31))
 (segment (start 114.5 130.009738) (end 114.5 130.759738) (width 0.25) (layer B.Cu) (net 31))
 (segment (start 114.25 129.109738) (end 114.25 129.759738) (width 0.25) (layer B.Cu) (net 31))
 (segment (start 115.25 128.759738) (end 114.6 128.759738) (width 0.25) (layer B.Cu) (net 31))
 (segment (start 114.6 128.759738) (end 114.25 129.109738) (width 0.25) (layer B.Cu) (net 31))
 (segment (start 119.25 128.259738) (end 120.75 128.259738) (width 0.25) (layer B.Cu) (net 1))
 (segment (start 120.75 128.259738) (end 121 128.009738) (width 0.25) (layer B.Cu) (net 1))
 (via (at 134.25 130) (size 1.2) (drill 0.7) (layers F.Cu B.Cu) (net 5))
 (segment (start 133.75 130) (end 134.25 130) (width 0.25) (layer B.Cu) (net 5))
 (segment (start 132.75 129) (end 133.75 130) (width 0.25) (layer B.Cu) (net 5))
 (segment (start 132.75 128.721002) (end 132.75 129) (width 0.25) (layer B.Cu) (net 5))
 (segment (start 132.75 128.170972) (end 132.75 128.721002) (width 0.25) (layer B.Cu) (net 5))
 (segment (start 132.120286 128.096258) (end 132.675286 128.096258) (width 0.25) (layer B.Cu) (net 5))
 (segment (start 132.675286 128.096258) (end 132.75 128.170972) (width 0.25) (layer B.Cu) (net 5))
 (segment (start 133.25 127) (end 133.75 127.5) (width 0.25) (layer B.Cu) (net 12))
 (segment (start 133.75 127.5) (end 133.75 128.5) (width 0.25) (layer B.Cu) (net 12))
 (via (at 133.75 128.5) (size 1.2) (drill 0.7) (layers F.Cu B.Cu) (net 12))
 (segment (start 132.36903 127) (end 133.25 127) (width 0.25) (layer B.Cu) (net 12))
 (segment (start 126.25 127) (end 132.36903 127) (width 0.25) (layer B.Cu) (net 12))
 (segment (start 126.120286 127.129714) (end 126.25 127) (width 0.25) (layer B.Cu) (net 12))
 (segment (start 126.120286 128.096258) (end 126.120286 127.129714) (width 0.25) (layer B.Cu) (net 12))
 (segment (start 123.109028 126.5) (end 134.25 126.5) (width 0.25) (layer B.Cu) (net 15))
 (via (at 134.25 126.5) (size 1.2) (drill 0.7) (layers F.Cu B.Cu) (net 15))
 (segment (start 122.310286 124.816258) (end 122.310286 125.701258) (width 0.25) (layer B.Cu) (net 15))
 (segment (start 122.310286 125.701258) (end 123.109028 126.5) (width 0.25) (layer B.Cu) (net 15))
 (segment (start 133.75 125) (end 133.75 124.5) (width 0.25) (layer B.Cu) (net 3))
 (via (at 133.75 124.5) (size 1.2) (drill 0.7) (layers F.Cu B.Cu) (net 3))
 (segment (start 133.75 125.5) (end 133.75 125) (width 0.25) (layer B.Cu) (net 3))
 (segment (start 133.25 126) (end 133.75 125.5) (width 0.25) (layer B.Cu) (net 3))
 (segment (start 128.609028 126) (end 133.25 126) (width 0.25) (layer B.Cu) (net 3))
 (segment (start 128.310286 124.816258) (end 128.310286 125.701258) (width 0.25) (layer B.Cu) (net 3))
 (segment (start 128.310286 125.701258) (end 128.609028 126) (width 0.25) (layer B.Cu) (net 3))
 (segment (start 114.25 126.759738) (end 113.5 127.509738) (width 0.25) (layer B.Cu) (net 25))
 (segment (start 115.25 126.759738) (end 114.25 126.759738) (width 0.25) (layer B.Cu) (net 25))
 (segment (start 115.25 127.259738) (end 114.5 127.259738) (width 0.25) (layer B.Cu) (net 26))
 (segment (start 114.5 127.259738) (end 113.75 128.009738) (width 0.25) (layer B.Cu) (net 26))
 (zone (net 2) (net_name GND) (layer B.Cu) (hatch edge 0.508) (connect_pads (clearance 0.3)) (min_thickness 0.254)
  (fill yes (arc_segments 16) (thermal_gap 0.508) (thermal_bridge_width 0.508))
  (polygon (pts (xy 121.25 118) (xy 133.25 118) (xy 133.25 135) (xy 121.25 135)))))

